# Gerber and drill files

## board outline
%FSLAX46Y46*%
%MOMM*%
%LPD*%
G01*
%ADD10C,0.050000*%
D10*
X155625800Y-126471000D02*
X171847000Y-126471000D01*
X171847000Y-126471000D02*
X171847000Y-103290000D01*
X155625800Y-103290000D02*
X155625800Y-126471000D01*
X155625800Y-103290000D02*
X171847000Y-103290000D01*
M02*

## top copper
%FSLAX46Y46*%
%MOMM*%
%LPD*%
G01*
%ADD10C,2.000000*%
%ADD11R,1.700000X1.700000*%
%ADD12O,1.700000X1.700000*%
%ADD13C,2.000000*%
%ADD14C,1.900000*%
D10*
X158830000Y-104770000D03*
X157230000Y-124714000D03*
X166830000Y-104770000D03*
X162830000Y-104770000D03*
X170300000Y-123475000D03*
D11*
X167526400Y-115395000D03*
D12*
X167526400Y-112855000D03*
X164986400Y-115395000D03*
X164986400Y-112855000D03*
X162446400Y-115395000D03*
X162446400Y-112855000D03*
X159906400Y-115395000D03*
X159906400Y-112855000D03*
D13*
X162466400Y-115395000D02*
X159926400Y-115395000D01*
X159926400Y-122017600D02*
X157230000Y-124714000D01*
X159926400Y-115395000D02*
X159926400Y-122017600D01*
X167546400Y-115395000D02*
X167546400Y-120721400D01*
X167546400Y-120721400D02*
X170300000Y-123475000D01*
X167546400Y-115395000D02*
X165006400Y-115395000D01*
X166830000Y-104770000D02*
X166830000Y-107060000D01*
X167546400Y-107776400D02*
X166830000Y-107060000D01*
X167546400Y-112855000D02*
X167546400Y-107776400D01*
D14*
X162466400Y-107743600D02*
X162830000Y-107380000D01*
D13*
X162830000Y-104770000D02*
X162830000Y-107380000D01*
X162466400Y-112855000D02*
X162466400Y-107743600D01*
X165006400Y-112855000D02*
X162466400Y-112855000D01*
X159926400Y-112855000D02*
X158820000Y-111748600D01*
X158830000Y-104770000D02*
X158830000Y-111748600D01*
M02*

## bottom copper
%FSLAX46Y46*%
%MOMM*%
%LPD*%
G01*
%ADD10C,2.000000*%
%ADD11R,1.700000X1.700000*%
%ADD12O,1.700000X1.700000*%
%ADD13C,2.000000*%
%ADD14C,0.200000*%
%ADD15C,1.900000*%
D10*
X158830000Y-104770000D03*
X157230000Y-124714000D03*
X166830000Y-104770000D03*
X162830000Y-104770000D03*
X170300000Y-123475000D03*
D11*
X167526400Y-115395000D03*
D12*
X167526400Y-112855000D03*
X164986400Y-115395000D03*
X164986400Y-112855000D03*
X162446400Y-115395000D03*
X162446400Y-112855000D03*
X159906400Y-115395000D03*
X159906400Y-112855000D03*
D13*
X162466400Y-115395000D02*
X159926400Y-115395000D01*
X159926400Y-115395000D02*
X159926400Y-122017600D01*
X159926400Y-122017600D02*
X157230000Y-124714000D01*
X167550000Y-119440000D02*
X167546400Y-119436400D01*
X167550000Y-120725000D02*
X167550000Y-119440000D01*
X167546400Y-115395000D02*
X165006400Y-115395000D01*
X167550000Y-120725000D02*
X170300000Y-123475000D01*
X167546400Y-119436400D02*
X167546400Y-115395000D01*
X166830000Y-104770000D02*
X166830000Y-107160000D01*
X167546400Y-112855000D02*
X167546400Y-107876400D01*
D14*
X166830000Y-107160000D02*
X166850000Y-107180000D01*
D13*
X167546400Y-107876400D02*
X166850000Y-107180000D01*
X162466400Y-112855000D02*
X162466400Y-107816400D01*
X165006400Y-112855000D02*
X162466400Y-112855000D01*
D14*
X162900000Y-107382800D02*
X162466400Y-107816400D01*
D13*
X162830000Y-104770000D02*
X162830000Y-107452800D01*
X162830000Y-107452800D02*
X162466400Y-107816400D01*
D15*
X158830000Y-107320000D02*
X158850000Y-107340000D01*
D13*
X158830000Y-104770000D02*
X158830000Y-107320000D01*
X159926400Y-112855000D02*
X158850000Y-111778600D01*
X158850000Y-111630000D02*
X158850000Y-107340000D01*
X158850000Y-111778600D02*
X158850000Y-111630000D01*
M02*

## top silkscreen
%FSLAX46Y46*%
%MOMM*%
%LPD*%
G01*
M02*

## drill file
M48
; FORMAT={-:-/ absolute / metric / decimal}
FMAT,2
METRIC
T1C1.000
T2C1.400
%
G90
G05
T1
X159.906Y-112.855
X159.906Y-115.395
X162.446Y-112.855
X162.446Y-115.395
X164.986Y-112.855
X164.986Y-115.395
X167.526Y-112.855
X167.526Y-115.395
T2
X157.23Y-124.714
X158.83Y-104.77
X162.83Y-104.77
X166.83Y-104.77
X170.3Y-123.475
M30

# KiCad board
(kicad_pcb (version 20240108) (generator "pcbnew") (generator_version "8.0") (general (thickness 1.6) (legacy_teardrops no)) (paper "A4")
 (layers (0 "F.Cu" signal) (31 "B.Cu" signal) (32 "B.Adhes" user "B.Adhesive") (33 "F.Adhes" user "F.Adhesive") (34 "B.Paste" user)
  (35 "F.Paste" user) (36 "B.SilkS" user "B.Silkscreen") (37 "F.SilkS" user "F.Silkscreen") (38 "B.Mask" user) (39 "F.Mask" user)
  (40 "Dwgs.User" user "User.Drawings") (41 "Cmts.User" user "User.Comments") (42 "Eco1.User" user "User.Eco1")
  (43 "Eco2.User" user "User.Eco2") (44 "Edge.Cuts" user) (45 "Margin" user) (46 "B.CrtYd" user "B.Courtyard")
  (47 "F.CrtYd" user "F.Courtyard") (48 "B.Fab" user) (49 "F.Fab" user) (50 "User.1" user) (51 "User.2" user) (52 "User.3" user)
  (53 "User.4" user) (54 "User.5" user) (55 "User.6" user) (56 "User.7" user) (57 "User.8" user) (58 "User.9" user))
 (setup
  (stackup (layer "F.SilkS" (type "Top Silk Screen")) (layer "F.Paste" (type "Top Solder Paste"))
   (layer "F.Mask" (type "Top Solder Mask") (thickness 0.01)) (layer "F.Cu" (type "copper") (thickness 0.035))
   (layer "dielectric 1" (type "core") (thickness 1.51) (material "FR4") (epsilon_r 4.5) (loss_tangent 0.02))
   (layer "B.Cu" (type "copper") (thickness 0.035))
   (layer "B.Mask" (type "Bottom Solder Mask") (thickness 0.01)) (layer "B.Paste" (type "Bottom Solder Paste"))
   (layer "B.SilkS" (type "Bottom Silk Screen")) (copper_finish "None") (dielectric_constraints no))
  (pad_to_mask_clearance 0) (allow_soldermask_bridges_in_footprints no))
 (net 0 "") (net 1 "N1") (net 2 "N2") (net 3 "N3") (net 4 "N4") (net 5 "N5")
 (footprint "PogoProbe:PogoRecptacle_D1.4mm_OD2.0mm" (layer "F.Cu") (at 158.83 104.77 90)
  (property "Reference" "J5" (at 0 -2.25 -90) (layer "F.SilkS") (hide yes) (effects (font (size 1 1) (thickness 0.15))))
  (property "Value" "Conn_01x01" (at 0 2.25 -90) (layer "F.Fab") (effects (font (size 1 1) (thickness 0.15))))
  (pad "1" thru_hole circle (at 0 0 90) (size 2 2) (drill 1.4) (layers "*.Cu" "*.Mask") (remove_unused_layers no) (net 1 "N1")))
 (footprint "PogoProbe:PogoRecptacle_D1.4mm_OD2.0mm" (layer "F.Cu") (at 157.23 124.714 90)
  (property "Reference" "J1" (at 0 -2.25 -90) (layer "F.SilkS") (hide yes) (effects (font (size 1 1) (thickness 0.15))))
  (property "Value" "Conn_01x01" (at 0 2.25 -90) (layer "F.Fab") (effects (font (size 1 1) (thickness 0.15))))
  (pad "1" thru_hole circle (at 0 0 90) (size 2 2) (drill 1.4) (layers "*.Cu" "*.Mask") (remove_unused_layers no) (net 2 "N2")))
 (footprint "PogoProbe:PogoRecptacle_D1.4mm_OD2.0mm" (layer "F.Cu") (at 166.83 104.77 90)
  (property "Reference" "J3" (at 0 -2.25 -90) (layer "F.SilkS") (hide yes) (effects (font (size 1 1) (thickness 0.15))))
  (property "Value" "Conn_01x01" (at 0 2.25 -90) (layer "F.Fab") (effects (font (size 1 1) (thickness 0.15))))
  (pad "1" thru_hole circle (at 0 0 90) (size 2 2) (drill 1.4) (layers "*.Cu" "*.Mask") (remove_unused_layers no) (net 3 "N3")))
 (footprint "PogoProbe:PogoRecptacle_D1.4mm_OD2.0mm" (layer "F.Cu") (at 162.83 104.77 90)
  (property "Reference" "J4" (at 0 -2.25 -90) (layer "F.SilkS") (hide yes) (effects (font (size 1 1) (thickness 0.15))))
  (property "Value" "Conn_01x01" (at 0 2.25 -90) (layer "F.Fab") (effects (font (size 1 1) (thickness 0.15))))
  (pad "1" thru_hole circle (at 0 0 90) (size 2 2) (drill 1.4) (layers "*.Cu" "*.Mask") (remove_unused_layers no) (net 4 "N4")))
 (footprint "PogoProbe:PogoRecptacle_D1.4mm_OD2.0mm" (layer "F.Cu") (at 170.3 123.475 90)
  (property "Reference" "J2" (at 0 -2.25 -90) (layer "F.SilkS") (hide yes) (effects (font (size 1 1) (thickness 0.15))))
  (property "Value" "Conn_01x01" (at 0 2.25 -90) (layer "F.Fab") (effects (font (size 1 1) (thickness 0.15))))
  (pad "1" thru_hole circle (at 0 0 90) (size 2 2) (drill 1.4) (layers "*.Cu" "*.Mask") (remove_unused_layers no) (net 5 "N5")))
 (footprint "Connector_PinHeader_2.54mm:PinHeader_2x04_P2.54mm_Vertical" (layer "B.Cu") (at 167.5264 115.395 90)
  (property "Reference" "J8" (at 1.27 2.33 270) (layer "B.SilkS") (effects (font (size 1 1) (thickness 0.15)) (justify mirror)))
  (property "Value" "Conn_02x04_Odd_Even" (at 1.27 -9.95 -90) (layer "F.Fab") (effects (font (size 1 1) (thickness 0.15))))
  (pad "1" thru_hole rect (at 0 0 90) (size 1.7 1.7) (drill 1) (layers "*.Cu" "*.Mask") (remove_unused_layers no) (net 5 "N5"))
  (pad "2" thru_hole oval (at 2.54 0 90) (size 1.7 1.7) (drill 1) (layers "*.Cu" "*.Mask") (remove_unused_layers no) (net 3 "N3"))
  (pad "3" thru_hole oval (at 0 -2.54 90) (size 1.7 1.7) (drill 1) (layers "*.Cu" "*.Mask") (remove_unused_layers no) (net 5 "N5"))
  (pad "4" thru_hole oval (at 2.54 -2.54 90) (size 1.7 1.7) (drill 1) (layers "*.Cu" "*.Mask") (remove_unused_layers no) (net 4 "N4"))
  (pad "5" thru_hole oval (at 0 -5.08 90) (size 1.7 1.7) (drill 1) (layers "*.Cu" "*.Mask") (remove_unused_layers no) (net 2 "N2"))
  (pad "6" thru_hole oval (at 2.54 -5.08 90) (size 1.7 1.7) (drill 1) (layers "*.Cu" "*.Mask") (remove_unused_layers no) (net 4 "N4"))
  (pad "7" thru_hole oval (at 0 -7.62 90) (size 1.7 1.7) (drill 1) (layers "*.Cu" "*.Mask") (remove_unused_layers no) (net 2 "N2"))
  (pad "8" thru_hole oval (at 2.54 -7.62 90) (size 1.7 1.7) (drill 1) (layers "*.Cu" "*.Mask") (remove_unused_layers no) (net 1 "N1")))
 (gr_line (start 155.6258 126.471) (end 171.847 126.471) (stroke (width 0.05) (type default)) (layer "Edge.Cuts"))
 (gr_line (start 171.847 126.471) (end 171.847 103.29) (stroke (width 0.05) (type default)) (layer "Edge.Cuts"))
 (gr_line (start 155.6258 103.29) (end 155.6258 126.471) (stroke (width 0.05) (type default)) (layer "Edge.Cuts"))
 (gr_line (start 155.6258 103.29) (end 171.847 103.29) (stroke (width 0.05) (type default)) (layer "Edge.Cuts"))
 (segment (start 162.4664 115.395) (end 159.9264 115.395) (width 2) (layer "F.Cu") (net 2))
 (segment (start 159.9264 122.0176) (end 157.23 124.714) (width 2) (layer "F.Cu") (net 2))
 (segment (start 159.9264 115.395) (end 159.9264 122.0176) (width 2) (layer "F.Cu") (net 2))
 (segment (start 162.4664 115.395) (end 159.9264 115.395) (width 2) (layer "B.Cu") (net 2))
 (segment (start 159.9264 115.395) (end 159.9264 122.0176) (width 2) (layer "B.Cu") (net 2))
 (segment (start 159.9264 122.0176) (end 157.23 124.714) (width 2) (layer "B.Cu") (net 2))
 (segment (start 167.5464 115.395) (end 167.5464 120.7214) (width 2) (layer "F.Cu") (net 5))
 (segment (start 167.5464 120.7214) (end 170.3 123.475) (width 2) (layer "F.Cu") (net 5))
 (segment (start 167.5464 115.395) (end 165.0064 115.395) (width 2) (layer "F.Cu") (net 5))
 (segment (start 167.55 119.44) (end 167.5464 119.4364) (width 2) (layer "B.Cu") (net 5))
 (segment (start 167.55 120.725) (end 167.55 119.44) (width 2) (layer "B.Cu") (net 5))
 (segment (start 167.5464 115.395) (end 165.0064 115.395) (width 2) (layer "B.Cu") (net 5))
 (segment (start 167.55 120.725) (end 170.3 123.475) (width 2) (layer "B.Cu") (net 5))
 (segment (start 167.5464 119.4364) (end 167.5464 115.395) (width 2) (layer "B.Cu") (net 5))
 (segment (start 166.83 104.77) (end 166.83 107.06) (width 2) (layer "F.Cu") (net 3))
 (segment (start 167.5464 107.7764) (end 166.83 107.06) (width 2) (layer "F.Cu") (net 3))
 (segment (start 167.5464 112.855) (end 167.5464 107.7764) (width 2) (layer "F.Cu") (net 3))
 (segment (start 166.83 104.77) (end 166.83 107.16) (width 2) (layer "B.Cu") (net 3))
 (segment (start 167.5464 112.855) (end 167.5464 107.8764) (width 2) (layer "B.Cu") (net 3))
 (segment (start 166.83 107.16) (end 166.85 107.18) (width 0.2) (layer "B.Cu") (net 3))
 (segment (start 167.5464 107.8764) (end 166.85 107.18) (width 2) (layer "B.Cu") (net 3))
 (segment (start 162.4664 107.7436) (end 162.83 107.38) (width 1.9) (layer "F.Cu") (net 4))
 (segment (start 162.83 104.77) (end 162.83 107.38) (width 2) (layer "F.Cu") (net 4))
 (segment (start 162.4664 112.855) (end 162.4664 107.7436) (width 2) (layer "F.Cu") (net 4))
 (segment (start 165.0064 112.855) (end 162.4664 112.855) (width 2) (layer "F.Cu") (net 4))
 (segment (start 162.4664 112.855) (end 162.4664 107.8164) (width 2) (layer "B.Cu") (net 4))
 (segment (start 165.0064 112.855) (end 162.4664 112.855) (width 2) (layer "B.Cu") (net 4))
 (segment (start 162.9 107.3828) (end 162.4664 107.8164) (width 0.2) (layer "B.Cu") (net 4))
 (segment (start 162.83 104.77) (end 162.83 107.4528) (width 2) (layer "B.Cu") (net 4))
 (segment (start 162.83 107.4528) (end 162.4664 107.8164) (width 2) (layer "B.Cu") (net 4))
 (segment (start 159.9264 112.855) (end 158.82 111.7486) (width 2) (layer "F.Cu") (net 1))
 (segment (start 158.83 104.77) (end 158.83 111.7486) (width 2) (layer "F.Cu") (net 1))
 (segment (start 158.83 107.32) (end 158.85 107.34) (width 1.9) (layer "B.Cu") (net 1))
 (segment (start 158.83 104.77) (end 158.83 107.32) (width 2) (layer "B.Cu") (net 1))
 (segment (start 159.9264 112.855) (end 158.85 111.7786) (width 2) (layer "B.Cu") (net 1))
 (segment (start 158.85 111.63) (end 158.85 107.34) (width 2) (layer "B.Cu") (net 1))
 (segment (start 158.85 111.7786) (end 158.85 111.63) (width 2) (layer "B.Cu") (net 1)))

